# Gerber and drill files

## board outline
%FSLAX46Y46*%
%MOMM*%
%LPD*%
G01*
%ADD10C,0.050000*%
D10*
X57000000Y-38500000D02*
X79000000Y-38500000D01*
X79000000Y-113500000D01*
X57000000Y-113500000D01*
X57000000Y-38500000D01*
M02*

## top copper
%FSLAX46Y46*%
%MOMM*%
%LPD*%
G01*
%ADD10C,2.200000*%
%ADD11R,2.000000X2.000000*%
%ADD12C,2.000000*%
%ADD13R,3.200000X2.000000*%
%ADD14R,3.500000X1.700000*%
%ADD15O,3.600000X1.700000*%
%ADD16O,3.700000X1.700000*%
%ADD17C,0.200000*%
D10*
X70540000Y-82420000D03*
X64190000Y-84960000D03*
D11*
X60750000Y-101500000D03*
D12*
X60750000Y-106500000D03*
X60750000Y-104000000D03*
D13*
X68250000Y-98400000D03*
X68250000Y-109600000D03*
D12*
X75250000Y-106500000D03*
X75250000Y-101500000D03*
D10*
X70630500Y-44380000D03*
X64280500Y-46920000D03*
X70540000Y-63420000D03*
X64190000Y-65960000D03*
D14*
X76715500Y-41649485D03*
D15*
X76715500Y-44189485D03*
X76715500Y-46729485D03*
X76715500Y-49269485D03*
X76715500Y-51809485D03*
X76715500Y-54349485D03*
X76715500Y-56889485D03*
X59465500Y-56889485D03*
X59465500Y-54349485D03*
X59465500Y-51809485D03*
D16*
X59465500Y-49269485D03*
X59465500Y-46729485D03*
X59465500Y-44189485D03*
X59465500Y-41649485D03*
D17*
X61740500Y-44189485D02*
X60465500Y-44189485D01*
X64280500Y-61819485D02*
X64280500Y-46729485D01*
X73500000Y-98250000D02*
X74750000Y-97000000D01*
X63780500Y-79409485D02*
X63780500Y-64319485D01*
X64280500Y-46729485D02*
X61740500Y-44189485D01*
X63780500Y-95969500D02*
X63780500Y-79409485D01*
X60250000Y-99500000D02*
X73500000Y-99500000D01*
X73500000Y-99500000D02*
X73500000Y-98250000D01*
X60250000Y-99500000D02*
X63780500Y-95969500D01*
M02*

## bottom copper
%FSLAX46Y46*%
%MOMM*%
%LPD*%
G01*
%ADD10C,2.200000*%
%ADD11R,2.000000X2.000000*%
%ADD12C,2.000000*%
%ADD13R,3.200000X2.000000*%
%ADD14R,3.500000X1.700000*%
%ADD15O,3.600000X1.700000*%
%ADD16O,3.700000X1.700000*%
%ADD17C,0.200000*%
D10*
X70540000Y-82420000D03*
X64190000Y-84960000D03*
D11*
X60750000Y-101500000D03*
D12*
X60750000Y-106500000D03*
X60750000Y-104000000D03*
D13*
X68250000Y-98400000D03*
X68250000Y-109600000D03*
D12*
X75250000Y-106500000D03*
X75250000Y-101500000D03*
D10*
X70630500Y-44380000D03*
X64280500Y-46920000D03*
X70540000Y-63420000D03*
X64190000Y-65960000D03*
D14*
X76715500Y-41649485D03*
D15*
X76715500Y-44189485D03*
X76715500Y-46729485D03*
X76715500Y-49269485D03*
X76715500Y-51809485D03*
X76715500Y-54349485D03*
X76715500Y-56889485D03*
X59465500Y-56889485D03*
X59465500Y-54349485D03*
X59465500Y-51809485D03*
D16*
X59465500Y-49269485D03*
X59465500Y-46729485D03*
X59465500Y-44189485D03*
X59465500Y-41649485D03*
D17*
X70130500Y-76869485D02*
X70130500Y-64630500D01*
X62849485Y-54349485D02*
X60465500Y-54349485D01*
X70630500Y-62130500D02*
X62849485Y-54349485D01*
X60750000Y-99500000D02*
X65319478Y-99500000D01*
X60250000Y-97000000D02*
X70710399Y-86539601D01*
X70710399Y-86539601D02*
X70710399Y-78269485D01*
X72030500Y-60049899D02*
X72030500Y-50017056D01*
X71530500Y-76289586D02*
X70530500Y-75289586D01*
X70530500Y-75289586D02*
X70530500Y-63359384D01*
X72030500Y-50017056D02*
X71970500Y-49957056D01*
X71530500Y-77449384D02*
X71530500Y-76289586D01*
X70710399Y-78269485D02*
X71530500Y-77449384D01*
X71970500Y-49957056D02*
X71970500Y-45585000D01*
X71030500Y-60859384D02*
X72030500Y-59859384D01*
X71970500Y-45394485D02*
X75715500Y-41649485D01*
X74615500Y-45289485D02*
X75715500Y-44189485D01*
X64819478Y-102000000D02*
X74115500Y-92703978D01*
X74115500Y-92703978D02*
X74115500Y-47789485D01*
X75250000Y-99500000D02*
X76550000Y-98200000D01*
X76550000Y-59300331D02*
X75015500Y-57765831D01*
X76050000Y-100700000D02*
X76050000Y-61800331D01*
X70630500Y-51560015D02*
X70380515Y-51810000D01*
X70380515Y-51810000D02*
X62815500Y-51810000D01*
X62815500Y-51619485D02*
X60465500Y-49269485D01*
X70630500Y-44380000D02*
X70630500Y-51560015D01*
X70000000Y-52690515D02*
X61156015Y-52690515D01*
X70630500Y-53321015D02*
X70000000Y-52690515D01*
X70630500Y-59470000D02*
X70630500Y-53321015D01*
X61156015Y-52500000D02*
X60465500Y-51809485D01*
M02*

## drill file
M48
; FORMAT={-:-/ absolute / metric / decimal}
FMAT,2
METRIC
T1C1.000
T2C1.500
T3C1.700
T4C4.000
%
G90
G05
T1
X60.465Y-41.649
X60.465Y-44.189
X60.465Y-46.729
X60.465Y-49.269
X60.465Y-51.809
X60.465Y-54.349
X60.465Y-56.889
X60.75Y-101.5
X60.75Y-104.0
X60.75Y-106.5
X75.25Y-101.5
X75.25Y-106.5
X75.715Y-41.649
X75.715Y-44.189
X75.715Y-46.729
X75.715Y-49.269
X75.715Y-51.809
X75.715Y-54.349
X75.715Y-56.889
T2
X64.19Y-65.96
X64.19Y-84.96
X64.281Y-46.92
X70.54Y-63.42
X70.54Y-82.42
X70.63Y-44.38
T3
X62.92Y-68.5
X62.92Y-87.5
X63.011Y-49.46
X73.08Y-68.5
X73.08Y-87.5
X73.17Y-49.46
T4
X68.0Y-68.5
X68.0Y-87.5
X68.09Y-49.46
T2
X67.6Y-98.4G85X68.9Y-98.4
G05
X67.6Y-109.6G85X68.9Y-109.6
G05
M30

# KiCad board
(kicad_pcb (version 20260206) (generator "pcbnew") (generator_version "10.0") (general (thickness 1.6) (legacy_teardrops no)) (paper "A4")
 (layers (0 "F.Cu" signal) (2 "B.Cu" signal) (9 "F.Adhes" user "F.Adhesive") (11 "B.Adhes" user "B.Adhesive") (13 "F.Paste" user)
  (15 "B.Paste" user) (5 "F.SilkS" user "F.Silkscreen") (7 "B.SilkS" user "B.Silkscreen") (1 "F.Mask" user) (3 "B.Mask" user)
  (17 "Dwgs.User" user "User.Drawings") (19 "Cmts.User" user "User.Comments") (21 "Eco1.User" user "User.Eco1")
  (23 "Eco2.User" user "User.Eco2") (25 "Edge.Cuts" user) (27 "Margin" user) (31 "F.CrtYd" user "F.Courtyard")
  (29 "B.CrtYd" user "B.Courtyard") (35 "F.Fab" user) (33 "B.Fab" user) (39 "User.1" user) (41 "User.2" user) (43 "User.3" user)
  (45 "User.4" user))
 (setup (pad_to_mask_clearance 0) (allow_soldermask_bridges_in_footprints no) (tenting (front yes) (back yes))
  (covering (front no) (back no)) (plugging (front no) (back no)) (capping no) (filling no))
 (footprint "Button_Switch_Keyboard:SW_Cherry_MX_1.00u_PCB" (layer "F.Cu") (at 70.54 82.42)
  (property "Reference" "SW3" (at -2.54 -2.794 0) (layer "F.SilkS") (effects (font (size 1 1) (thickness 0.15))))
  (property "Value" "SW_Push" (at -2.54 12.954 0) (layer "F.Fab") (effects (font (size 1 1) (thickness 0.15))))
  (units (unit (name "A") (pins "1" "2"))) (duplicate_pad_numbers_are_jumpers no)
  (pad "" np_thru_hole circle (at -7.62 5.08) (size 1.7 1.7) (drill 1.7) (layers "*.Cu" "*.Mask"))
  (pad "" np_thru_hole circle (at -2.54 5.08) (size 4 4) (drill 4) (layers "*.Cu" "*.Mask"))
  (pad "" np_thru_hole circle (at 2.54 5.08) (size 1.7 1.7) (drill 1.7) (layers "*.Cu" "*.Mask"))
  (pad "1" thru_hole circle (at 0 0) (size 2.2 2.2) (drill 1.5) (layers "*.Cu" "*.Mask") (remove_unused_layers no)
   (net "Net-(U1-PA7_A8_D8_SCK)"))
  (pad "2" thru_hole circle (at -6.35 2.54) (size 2.2 2.2) (drill 1.5) (layers "*.Cu" "*.Mask") (remove_unused_layers no) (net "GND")))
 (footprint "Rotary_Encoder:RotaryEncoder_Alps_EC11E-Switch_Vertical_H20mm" (layer "F.Cu") (at 60.75 101.5)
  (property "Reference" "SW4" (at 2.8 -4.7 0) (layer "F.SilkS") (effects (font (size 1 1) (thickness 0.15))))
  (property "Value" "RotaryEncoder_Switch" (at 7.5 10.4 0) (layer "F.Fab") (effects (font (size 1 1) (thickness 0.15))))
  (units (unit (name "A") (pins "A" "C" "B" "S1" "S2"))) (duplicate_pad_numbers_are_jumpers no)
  (pad "A" thru_hole rect (at 0 0) (size 2 2) (drill 1) (layers "*.Cu" "*.Mask") (remove_unused_layers no) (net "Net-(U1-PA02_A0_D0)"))
  (pad "B" thru_hole circle (at 0 5) (size 2 2) (drill 1) (layers "*.Cu" "*.Mask") (remove_unused_layers no) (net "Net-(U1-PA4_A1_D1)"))
  (pad "C" thru_hole circle (at 0 2.5) (size 2 2) (drill 1) (layers "*.Cu" "*.Mask") (remove_unused_layers no) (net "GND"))
  (pad "MP" thru_hole rect (at 7.5 -3.1) (size 3.2 2) (drill oval 2.8 1.5) (layers "*.Cu" "*.Mask") (remove_unused_layers no))
  (pad "MP" thru_hole rect (at 7.5 8.1) (size 3.2 2) (drill oval 2.8 1.5) (layers "*.Cu" "*.Mask") (remove_unused_layers no))
  (pad "S1" thru_hole circle (at 14.5 5) (size 2 2) (drill 1) (layers "*.Cu" "*.Mask") (remove_unused_layers no) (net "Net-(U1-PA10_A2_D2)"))
  (pad "S2" thru_hole circle (at 14.5 0) (size 2 2) (drill 1) (layers "*.Cu" "*.Mask") (remove_unused_layers no) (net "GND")))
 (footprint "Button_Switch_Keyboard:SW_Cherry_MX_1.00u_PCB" (layer "F.Cu") (at 70.6305 44.38)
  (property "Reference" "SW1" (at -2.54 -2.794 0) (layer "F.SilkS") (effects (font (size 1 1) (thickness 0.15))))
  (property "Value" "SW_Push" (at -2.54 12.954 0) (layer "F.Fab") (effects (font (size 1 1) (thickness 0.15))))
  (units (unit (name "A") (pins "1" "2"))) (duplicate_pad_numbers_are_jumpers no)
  (pad "" np_thru_hole circle (at -7.62 5.08) (size 1.7 1.7) (drill 1.7) (layers "*.Cu" "*.Mask"))
  (pad "" np_thru_hole circle (at -2.54 5.08) (size 4 4) (drill 4) (layers "*.Cu" "*.Mask"))
  (pad "" np_thru_hole circle (at 2.54 5.08) (size 1.7 1.7) (drill 1.7) (layers "*.Cu" "*.Mask"))
  (pad "1" thru_hole circle (at 0 0) (size 2.2 2.2) (drill 1.5) (layers "*.Cu" "*.Mask") (remove_unused_layers no)
   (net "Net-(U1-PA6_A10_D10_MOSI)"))
  (pad "2" thru_hole circle (at -6.35 2.54) (size 2.2 2.2) (drill 1.5) (layers "*.Cu" "*.Mask") (remove_unused_layers no) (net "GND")))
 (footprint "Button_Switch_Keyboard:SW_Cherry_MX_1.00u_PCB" (layer "F.Cu") (at 70.54 63.42)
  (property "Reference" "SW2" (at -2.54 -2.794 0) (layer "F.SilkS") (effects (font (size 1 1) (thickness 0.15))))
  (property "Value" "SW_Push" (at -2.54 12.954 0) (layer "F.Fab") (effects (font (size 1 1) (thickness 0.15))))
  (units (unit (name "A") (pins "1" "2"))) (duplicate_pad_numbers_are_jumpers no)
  (pad "" np_thru_hole circle (at -7.62 5.08) (size 1.7 1.7) (drill 1.7) (layers "*.Cu" "*.Mask"))
  (pad "" np_thru_hole circle (at -2.54 5.08) (size 4 4) (drill 4) (layers "*.Cu" "*.Mask"))
  (pad "" np_thru_hole circle (at 2.54 5.08) (size 1.7 1.7) (drill 1.7) (layers "*.Cu" "*.Mask"))
  (pad "1" thru_hole circle (at 0 0) (size 2.2 2.2) (drill 1.5) (layers "*.Cu" "*.Mask") (remove_unused_layers no)
   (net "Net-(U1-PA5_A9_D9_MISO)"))
  (pad "2" thru_hole circle (at -6.35 2.54) (size 2.2 2.2) (drill 1.5) (layers "*.Cu" "*.Mask") (remove_unused_layers no) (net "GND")))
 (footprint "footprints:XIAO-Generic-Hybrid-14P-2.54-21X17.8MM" (layer "B.Cu") (at 68.0905 49.269485 180)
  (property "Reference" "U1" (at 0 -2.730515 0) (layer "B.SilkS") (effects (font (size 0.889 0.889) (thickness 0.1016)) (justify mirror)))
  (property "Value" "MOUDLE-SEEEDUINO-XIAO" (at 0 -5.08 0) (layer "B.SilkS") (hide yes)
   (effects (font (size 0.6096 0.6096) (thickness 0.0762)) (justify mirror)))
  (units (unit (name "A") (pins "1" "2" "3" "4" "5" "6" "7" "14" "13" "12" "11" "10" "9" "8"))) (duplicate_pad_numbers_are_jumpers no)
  (pad "1" thru_hole rect (at -7.625 7.62 180) (size 3.5 1.7) (drill 1 (offset -1 0)) (layers "*.Cu" "*.Mask") (remove_unused_layers no)
   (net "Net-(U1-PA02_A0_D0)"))
  (pad "2" thru_hole oval (at -7.625 5.08 180) (size 3.6 1.7) (drill 1 (offset -1 0)) (layers "*.Cu" "*.Mask") (remove_unused_layers no)
   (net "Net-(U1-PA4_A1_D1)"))
  (pad "3" thru_hole oval (at -7.625 2.54 180) (size 3.6 1.7) (drill 1 (offset -1 0)) (layers "*.Cu" "*.Mask") (remove_unused_layers no)
   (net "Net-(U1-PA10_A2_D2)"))
  (pad "4" thru_hole oval (at -7.625 0 180) (size 3.6 1.7) (drill 1 (offset -1 0)) (layers "*.Cu" "*.Mask") (remove_unused_layers no)
   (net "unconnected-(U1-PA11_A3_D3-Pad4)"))
  (pad "5" thru_hole oval (at -7.625 -2.54 180) (size 3.6 1.7) (drill 1 (offset -1 0)) (layers "*.Cu" "*.Mask") (remove_unused_layers no)
   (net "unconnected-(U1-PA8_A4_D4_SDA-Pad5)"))
  (pad "6" thru_hole oval (at -7.625 -5.08) (size 3.6 1.7) (drill 1 (offset 1 0)) (layers "*.Cu" "*.Mask") (remove_unused_layers no)
   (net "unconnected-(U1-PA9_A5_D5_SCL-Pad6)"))
  (pad "7" thru_hole oval (at -7.625 -7.62 180) (size 3.6 1.7) (drill 1 (offset -1 0)) (layers "*.Cu" "*.Mask") (remove_unused_layers no)
   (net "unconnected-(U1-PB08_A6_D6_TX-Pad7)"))
  (pad "8" thru_hole oval (at 7.625 -7.62 180) (size 3.6 1.7) (drill 1 (offset 1 0)) (layers "*.Cu" "*.Mask") (remove_unused_layers no)
   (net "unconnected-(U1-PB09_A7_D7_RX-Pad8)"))
  (pad "9" thru_hole oval (at 7.625 -5.08 180) (size 3.6 1.7) (drill 1 (offset 1 0)) (layers "*.Cu" "*.Mask") (remove_unused_layers no)
   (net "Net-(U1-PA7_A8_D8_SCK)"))
  (pad "10" thru_hole oval (at 7.625 -2.54 180) (size 3.6 1.7) (drill 1 (offset 1 0)) (layers "*.Cu" "*.Mask") (remove_unused_layers no)
   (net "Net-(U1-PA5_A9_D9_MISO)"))
  (pad "11" thru_hole oval (at 7.625 0 180) (size 3.7 1.7) (drill 1 (offset 1 0)) (layers "*.Cu" "*.Mask") (remove_unused_layers no)
   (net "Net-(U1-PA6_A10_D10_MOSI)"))
  (pad "12" thru_hole oval (at 7.625 2.54 180) (size 3.7 1.7) (drill 1 (offset 1 0)) (layers "*.Cu" "*.Mask") (remove_unused_layers no)
   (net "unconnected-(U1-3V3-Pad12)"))
  (pad "13" thru_hole oval (at 7.625 5.08 180) (size 3.7 1.7) (drill 1 (offset 1 0)) (layers "*.Cu" "*.Mask") (remove_unused_layers no)
   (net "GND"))
  (pad "14" thru_hole oval (at 7.625 7.62 180) (size 3.7 1.7) (drill 1 (offset 1 0)) (layers "*.Cu" "*.Mask") (remove_unused_layers no)
   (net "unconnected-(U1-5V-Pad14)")))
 (gr_rect (start 57 38.5) (end 79 113.5) (stroke (width 0.05) (type default)) (fill no) (layer "Edge.Cuts"))
 (segment (start 70.1305 76.869485) (end 70.1305 64.6305) (width 0.2) (layer "B.Cu") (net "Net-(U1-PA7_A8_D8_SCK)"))
 (segment (start 62.849485 54.349485) (end 60.4655 54.349485) (width 0.2) (layer "B.Cu") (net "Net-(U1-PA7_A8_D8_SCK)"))
 (segment (start 70.6305 62.1305) (end 62.849485 54.349485) (width 0.2) (layer "B.Cu") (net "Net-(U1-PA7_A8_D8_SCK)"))
 (segment (start 61.7405 44.189485) (end 60.4655 44.189485) (width 0.2) (layer "F.Cu") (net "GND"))
 (segment (start 64.2805 61.819485) (end 64.2805 46.729485) (width 0.2) (layer "F.Cu") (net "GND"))
 (segment (start 73.5 98.25) (end 74.75 97) (width 0.2) (layer "F.Cu") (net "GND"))
 (segment (start 63.7805 79.409485) (end 63.7805 64.319485) (width 0.2) (layer "F.Cu") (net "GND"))
 (segment (start 64.2805 46.729485) (end 61.7405 44.189485) (width 0.2) (layer "F.Cu") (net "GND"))
 (segment (start 63.7805 95.9695) (end 63.7805 79.409485) (width 0.2) (layer "F.Cu") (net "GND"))
 (segment (start 60.25 99.5) (end 73.5 99.5) (width 0.2) (layer "F.Cu") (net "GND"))
 (segment (start 73.5 99.5) (end 73.5 98.25) (width 0.2) (layer "F.Cu") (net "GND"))
 (segment (start 60.25 99.5) (end 63.7805 95.9695) (width 0.2) (layer "F.Cu") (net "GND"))
 (segment (start 60.75 99.5) (end 65.319478 99.5) (width 0.2) (layer "B.Cu") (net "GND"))
 (segment (start 60.25 97) (end 70.710399 86.539601) (width 0.2) (layer "B.Cu") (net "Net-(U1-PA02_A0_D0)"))
 (segment (start 70.710399 86.539601) (end 70.710399 78.269485) (width 0.2) (layer "B.Cu") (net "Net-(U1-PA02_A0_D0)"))
 (segment (start 72.0305 60.049899) (end 72.0305 50.017056) (width 0.2) (layer "B.Cu") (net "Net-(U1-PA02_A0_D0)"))
 (segment (start 71.5305 76.289586) (end 70.5305 75.289586) (width 0.2) (layer "B.Cu") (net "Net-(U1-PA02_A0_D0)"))
 (segment (start 70.5305 75.289586) (end 70.5305 63.359384) (width 0.2) (layer "B.Cu") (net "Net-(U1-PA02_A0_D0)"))
 (segment (start 72.0305 50.017056) (end 71.9705 49.957056) (width 0.2) (layer "B.Cu") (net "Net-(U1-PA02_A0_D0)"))
 (segment (start 71.5305 77.449384) (end 71.5305 76.289586) (width 0.2) (layer "B.Cu") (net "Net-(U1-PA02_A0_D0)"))
 (segment (start 70.710399 78.269485) (end 71.5305 77.449384) (width 0.2) (layer "B.Cu") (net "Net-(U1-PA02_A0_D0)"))
 (segment (start 71.9705 49.957056) (end 71.9705 45.585) (width 0.2) (layer "B.Cu") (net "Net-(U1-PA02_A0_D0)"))
 (segment (start 71.0305 60.859384) (end 72.0305 59.859384) (width 0.2) (layer "B.Cu") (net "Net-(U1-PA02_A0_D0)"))
 (segment (start 71.9705 45.394485) (end 75.7155 41.649485) (width 0.2) (layer "B.Cu") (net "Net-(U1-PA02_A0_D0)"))
 (segment (start 74.6155 45.289485) (end 75.7155 44.189485) (width 0.2) (layer "B.Cu") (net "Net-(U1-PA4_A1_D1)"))
 (segment (start 64.819478 102) (end 74.1155 92.703978) (width 0.2) (layer "B.Cu") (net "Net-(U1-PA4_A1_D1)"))
 (segment (start 74.1155 92.703978) (end 74.1155 47.789485) (width 0.2) (layer "B.Cu") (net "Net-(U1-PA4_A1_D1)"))
 (segment (start 75.25 99.5) (end 76.55 98.2) (width 0.2) (layer "B.Cu") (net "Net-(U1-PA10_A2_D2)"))
 (segment (start 76.55 59.300331) (end 75.0155 57.765831) (width 0.2) (layer "B.Cu") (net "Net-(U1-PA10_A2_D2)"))
 (segment (start 76.05 100.7) (end 76.05 61.800331) (width 0.2) (layer "B.Cu") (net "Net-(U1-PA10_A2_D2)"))
 (segment (start 70.6305 51.560015) (end 70.380515 51.81) (width 0.2) (layer "B.Cu") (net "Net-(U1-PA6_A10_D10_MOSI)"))
 (segment (start 70.380515 51.81) (end 62.8155 51.81) (width 0.2) (layer "B.Cu") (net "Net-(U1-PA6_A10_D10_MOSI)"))
 (segment (start 62.8155 51.619485) (end 60.4655 49.269485) (width 0.2) (layer "B.Cu") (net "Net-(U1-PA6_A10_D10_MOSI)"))
 (segment (start 70.6305 44.38) (end 70.6305 51.560015) (width 0.2) (layer "B.Cu") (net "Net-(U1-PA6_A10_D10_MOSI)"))
 (segment (start 70 52.690515) (end 61.156015 52.690515) (width 0.2) (layer "B.Cu") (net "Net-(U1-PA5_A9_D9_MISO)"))
 (segment (start 70.6305 53.321015) (end 70 52.690515) (width 0.2) (layer "B.Cu") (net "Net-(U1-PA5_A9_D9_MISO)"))
 (segment (start 70.6305 59.47) (end 70.6305 53.321015) (width 0.2) (layer "B.Cu") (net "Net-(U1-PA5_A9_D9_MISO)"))
 (segment (start 61.156015 52.5) (end 60.4655 51.809485) (width 0.2) (layer "B.Cu") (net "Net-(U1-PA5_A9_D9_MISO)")))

